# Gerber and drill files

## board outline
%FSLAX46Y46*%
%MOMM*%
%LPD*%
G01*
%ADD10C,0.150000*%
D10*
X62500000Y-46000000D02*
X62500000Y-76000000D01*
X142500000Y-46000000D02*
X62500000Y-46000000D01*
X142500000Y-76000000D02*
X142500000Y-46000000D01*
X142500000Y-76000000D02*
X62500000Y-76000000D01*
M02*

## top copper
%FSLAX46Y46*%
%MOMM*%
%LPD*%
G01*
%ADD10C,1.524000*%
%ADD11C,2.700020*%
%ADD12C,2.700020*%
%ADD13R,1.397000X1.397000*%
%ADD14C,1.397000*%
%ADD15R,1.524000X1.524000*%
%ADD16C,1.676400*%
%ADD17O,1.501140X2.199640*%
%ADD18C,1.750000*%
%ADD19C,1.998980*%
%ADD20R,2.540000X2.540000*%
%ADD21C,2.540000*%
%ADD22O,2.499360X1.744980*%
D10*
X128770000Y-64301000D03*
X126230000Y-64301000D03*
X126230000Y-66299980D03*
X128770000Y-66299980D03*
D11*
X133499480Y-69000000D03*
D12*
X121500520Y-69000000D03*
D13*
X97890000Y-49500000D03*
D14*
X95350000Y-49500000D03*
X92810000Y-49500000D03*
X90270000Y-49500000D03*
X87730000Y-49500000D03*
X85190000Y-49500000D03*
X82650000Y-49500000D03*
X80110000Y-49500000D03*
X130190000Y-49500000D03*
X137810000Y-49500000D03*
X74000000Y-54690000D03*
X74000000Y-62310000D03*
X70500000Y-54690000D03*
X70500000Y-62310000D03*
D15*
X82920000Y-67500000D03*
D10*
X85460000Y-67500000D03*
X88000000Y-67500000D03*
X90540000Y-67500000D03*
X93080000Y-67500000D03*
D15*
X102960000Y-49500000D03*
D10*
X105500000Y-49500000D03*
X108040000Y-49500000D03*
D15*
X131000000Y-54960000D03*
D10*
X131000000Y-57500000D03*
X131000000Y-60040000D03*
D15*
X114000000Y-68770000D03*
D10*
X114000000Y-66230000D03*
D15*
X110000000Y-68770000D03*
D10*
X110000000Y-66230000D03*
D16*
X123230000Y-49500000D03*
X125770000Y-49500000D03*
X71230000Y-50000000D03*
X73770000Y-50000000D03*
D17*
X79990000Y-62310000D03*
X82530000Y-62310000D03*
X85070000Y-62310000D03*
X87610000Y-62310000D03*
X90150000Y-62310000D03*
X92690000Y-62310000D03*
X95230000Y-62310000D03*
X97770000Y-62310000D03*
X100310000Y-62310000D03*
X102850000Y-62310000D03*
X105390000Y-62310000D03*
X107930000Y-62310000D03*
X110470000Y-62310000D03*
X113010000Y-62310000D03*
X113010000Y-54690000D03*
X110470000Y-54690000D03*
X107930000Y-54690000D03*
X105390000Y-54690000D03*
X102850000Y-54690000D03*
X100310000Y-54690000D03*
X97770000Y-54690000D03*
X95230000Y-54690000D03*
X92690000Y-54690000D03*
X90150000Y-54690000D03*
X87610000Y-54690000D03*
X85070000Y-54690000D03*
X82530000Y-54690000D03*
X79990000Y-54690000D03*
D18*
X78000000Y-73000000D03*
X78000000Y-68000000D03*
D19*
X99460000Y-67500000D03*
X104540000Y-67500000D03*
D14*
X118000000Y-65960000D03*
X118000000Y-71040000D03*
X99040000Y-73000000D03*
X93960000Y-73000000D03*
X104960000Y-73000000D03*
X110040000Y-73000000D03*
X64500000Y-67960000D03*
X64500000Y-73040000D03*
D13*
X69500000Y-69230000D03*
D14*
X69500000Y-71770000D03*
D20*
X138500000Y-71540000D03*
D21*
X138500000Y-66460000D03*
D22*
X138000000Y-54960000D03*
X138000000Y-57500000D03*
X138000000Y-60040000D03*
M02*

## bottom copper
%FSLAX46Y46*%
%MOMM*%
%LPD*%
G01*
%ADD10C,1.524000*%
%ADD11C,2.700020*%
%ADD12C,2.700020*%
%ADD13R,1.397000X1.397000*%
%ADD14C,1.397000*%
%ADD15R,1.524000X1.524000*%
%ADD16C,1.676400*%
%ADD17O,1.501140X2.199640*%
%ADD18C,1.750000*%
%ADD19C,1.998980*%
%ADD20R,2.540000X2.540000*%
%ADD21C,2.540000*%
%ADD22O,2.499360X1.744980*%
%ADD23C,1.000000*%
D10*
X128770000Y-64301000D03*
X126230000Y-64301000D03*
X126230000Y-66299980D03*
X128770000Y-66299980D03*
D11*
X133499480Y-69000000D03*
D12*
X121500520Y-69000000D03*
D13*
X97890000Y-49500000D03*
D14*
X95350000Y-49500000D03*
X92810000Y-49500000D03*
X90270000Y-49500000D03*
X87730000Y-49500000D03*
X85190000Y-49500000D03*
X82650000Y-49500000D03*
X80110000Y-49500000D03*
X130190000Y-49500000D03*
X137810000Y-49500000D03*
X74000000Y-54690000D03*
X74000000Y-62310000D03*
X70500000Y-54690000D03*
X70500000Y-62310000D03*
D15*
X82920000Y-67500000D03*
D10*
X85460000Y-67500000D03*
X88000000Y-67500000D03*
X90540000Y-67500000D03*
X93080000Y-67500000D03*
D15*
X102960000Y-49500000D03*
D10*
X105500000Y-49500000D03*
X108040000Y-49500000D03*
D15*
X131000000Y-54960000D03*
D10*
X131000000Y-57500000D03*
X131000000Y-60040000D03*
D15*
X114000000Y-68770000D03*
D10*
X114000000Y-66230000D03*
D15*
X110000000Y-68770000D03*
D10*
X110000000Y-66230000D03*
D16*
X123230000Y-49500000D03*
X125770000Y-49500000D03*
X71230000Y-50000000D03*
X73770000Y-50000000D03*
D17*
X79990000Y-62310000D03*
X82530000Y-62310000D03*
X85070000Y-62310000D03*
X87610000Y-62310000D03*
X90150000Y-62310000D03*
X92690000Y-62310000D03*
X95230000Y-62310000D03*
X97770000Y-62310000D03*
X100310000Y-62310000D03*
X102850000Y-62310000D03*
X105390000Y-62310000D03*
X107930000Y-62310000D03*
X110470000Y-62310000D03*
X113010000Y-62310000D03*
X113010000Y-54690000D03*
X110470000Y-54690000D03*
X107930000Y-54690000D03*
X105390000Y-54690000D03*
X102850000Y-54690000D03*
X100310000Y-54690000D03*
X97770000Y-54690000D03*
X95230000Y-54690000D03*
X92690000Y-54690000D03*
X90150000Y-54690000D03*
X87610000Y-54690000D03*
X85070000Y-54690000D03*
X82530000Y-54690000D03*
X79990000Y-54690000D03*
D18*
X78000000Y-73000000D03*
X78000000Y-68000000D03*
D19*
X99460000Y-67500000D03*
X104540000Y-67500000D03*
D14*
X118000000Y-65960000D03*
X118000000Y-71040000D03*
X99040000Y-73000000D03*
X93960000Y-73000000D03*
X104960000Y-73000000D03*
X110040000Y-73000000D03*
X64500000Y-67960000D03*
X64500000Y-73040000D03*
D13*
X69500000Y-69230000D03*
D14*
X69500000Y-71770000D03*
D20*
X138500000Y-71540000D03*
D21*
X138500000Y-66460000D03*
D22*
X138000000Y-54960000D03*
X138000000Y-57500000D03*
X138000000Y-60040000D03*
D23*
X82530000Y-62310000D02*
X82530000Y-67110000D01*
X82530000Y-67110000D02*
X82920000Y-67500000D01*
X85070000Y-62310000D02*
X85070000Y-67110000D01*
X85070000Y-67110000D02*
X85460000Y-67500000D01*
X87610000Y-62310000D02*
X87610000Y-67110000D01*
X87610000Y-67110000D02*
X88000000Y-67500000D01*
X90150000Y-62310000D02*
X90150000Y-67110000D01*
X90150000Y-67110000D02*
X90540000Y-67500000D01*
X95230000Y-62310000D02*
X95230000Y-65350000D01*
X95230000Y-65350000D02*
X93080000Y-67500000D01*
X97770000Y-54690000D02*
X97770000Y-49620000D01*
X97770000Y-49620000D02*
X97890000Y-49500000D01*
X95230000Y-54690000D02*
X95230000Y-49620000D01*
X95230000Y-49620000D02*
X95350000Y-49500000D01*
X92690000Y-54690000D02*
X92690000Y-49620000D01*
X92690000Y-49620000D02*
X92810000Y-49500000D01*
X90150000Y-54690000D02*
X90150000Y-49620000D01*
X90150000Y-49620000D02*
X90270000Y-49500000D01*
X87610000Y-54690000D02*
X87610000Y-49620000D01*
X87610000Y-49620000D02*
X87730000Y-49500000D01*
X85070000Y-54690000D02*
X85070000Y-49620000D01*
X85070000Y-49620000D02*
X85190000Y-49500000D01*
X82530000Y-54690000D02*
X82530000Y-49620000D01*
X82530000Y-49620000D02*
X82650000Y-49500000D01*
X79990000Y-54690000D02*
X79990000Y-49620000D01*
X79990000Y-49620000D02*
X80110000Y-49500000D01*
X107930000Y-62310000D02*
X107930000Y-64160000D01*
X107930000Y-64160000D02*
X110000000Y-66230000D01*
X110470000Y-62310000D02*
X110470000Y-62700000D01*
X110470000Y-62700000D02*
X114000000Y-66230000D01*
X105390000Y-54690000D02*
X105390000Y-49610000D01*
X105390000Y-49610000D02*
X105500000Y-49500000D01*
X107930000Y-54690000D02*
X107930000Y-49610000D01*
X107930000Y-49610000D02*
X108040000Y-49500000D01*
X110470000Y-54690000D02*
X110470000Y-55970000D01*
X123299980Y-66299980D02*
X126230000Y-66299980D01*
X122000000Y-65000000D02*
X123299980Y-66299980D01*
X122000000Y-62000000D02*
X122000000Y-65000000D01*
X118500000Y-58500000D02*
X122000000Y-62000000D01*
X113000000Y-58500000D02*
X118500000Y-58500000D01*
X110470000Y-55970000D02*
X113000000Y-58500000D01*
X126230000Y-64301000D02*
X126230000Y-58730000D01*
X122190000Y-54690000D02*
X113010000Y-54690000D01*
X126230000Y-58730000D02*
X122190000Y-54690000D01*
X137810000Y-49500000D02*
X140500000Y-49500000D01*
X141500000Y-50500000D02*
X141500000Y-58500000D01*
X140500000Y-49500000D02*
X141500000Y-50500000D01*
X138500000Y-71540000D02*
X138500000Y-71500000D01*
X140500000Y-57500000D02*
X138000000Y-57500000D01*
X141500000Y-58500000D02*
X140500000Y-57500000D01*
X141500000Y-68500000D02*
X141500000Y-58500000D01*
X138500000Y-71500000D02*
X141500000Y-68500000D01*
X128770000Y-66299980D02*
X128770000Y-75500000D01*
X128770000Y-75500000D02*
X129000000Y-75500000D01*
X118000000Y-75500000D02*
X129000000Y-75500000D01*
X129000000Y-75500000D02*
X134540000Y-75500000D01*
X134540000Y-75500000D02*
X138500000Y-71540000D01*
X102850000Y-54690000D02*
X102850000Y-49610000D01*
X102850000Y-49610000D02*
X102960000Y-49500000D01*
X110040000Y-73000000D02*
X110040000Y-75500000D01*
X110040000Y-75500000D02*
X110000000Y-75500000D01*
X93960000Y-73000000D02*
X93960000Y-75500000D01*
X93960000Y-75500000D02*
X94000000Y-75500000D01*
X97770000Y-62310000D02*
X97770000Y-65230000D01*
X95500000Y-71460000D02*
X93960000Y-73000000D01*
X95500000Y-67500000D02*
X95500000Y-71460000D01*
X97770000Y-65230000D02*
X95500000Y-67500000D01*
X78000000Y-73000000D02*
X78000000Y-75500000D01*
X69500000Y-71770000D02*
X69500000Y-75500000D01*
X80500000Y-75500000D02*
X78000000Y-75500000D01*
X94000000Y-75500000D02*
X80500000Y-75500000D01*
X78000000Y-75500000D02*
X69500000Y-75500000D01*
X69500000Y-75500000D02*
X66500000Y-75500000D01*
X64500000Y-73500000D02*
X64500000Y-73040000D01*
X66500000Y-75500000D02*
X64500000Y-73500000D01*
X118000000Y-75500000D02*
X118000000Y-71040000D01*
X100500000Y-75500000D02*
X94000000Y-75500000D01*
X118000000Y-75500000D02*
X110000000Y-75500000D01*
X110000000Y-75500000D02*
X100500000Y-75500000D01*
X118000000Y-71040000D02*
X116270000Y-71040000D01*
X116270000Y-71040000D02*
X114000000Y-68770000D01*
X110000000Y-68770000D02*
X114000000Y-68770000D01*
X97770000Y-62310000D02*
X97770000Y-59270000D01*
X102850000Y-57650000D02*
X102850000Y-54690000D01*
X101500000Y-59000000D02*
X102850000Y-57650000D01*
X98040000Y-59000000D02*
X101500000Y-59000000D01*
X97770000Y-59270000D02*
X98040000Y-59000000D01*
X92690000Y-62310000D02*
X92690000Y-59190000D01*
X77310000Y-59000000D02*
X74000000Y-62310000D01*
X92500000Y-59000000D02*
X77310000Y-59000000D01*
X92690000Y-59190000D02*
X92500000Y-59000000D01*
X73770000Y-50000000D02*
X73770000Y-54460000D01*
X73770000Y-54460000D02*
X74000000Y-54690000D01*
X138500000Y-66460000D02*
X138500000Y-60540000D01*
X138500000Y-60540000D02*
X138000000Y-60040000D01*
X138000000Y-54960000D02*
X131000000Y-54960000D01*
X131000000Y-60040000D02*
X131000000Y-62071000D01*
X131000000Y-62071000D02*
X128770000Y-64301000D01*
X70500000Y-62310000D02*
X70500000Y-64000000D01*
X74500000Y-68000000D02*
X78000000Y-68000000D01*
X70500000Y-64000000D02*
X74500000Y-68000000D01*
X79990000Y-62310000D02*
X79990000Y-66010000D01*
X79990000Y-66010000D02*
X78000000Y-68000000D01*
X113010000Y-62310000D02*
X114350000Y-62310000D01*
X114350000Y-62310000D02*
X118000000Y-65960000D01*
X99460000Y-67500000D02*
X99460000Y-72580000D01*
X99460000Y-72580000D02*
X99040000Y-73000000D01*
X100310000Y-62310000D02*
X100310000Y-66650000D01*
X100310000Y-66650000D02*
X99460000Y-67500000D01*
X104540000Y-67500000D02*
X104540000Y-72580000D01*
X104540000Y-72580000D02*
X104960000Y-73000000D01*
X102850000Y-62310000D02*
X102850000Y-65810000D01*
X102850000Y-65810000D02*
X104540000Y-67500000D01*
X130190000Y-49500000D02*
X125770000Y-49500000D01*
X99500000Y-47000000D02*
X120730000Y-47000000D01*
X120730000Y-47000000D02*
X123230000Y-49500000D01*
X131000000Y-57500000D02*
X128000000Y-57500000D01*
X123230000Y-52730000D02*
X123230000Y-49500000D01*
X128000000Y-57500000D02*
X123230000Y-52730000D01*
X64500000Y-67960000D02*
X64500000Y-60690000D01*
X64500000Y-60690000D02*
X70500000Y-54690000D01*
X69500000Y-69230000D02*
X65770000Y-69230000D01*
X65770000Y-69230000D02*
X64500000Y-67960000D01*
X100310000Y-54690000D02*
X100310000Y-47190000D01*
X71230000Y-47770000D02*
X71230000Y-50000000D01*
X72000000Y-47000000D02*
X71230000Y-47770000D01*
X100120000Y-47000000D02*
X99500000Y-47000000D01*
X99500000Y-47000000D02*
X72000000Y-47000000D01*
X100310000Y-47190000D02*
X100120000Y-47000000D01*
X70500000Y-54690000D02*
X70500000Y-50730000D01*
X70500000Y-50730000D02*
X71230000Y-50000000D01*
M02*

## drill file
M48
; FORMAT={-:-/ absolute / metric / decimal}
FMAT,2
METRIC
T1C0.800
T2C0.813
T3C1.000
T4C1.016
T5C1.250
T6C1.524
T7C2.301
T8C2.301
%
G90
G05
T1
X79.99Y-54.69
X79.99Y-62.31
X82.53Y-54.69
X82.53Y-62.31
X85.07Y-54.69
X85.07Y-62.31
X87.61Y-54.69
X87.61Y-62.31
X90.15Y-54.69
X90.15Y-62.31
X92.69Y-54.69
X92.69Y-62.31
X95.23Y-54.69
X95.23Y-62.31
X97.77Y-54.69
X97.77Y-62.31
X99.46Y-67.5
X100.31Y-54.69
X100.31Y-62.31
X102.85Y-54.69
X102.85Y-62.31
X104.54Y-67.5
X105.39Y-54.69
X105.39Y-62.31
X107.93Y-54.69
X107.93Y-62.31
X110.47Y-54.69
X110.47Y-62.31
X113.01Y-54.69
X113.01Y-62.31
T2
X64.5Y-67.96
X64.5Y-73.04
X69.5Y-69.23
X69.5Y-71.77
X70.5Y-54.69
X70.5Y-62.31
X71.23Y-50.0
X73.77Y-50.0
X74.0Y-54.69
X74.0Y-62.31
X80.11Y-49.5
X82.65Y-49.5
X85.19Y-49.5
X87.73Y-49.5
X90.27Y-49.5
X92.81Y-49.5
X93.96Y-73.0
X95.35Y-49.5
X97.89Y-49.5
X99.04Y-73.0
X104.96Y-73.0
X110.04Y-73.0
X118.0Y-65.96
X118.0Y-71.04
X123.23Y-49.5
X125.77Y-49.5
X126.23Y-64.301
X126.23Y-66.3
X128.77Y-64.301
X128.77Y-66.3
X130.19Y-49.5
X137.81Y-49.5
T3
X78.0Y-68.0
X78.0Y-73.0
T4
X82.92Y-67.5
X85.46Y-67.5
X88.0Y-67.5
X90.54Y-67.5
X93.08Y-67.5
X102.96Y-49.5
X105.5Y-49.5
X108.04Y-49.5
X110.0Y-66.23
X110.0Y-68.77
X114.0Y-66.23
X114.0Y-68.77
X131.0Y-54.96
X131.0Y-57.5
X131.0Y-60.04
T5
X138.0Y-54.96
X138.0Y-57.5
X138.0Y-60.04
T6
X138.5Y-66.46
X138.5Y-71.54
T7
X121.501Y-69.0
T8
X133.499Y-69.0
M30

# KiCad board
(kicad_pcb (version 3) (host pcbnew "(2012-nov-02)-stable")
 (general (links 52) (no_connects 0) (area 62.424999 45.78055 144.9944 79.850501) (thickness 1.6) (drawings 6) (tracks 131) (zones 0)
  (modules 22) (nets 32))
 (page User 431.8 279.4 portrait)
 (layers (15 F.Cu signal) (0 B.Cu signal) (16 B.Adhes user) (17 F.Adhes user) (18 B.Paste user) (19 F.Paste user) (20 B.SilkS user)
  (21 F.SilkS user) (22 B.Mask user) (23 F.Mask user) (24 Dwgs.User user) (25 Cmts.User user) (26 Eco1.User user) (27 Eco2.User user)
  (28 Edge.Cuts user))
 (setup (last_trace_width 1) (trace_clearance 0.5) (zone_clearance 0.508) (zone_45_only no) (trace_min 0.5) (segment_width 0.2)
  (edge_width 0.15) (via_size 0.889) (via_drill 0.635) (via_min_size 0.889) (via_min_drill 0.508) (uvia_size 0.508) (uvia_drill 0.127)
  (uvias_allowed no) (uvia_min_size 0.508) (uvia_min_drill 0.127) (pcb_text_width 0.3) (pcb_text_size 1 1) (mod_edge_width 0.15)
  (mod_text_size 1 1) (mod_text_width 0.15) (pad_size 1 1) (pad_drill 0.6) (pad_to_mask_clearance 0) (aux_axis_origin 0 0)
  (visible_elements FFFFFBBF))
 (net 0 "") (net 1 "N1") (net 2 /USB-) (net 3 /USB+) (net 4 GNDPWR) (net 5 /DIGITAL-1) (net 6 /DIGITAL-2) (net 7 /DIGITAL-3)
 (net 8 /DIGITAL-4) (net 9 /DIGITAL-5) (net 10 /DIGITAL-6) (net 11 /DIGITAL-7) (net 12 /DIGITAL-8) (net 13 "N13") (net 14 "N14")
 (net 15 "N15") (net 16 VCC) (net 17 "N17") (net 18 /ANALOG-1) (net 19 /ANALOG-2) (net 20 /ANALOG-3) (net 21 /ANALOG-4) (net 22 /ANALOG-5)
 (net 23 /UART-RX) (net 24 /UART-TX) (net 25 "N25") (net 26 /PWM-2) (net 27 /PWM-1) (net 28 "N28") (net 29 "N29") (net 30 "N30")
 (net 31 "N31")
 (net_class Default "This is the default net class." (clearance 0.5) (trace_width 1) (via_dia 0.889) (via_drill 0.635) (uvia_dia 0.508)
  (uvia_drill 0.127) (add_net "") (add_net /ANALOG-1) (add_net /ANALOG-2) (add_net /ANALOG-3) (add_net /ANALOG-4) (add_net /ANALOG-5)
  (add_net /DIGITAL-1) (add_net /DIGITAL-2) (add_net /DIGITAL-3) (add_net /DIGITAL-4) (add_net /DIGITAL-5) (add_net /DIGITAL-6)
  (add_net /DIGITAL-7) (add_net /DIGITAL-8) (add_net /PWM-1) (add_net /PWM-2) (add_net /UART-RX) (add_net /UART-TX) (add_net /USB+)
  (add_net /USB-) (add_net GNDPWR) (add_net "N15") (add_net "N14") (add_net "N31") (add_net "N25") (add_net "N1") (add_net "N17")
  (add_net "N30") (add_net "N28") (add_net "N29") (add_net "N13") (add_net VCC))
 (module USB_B (layer F.Cu) (at 127.5 69)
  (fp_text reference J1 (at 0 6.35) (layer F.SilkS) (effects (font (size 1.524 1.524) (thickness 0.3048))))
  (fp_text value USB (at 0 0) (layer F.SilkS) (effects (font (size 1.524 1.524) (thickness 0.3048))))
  (pad 1 thru_hole circle (at 1.27 -4.699) (size 1.524 1.524) (drill 0.8128) (layers *.Cu *.Mask F.SilkS) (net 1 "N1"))
  (pad 2 thru_hole circle (at -1.27 -4.699) (size 1.524 1.524) (drill 0.8128) (layers *.Cu *.Mask F.SilkS) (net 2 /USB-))
  (pad 3 thru_hole circle (at -1.27 -2.70002) (size 1.524 1.524) (drill 0.8128) (layers *.Cu *.Mask F.SilkS) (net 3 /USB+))
  (pad 4 thru_hole circle (at 1.27 -2.70002) (size 1.524 1.524) (drill 0.8128) (layers *.Cu *.Mask F.SilkS) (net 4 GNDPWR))
  (pad 5 np_thru_hole circle (at 5.99948 0) (size 2.70002 2.70002) (drill 2.30124) (layers *.Cu *.SilkS *.Mask))
  (pad 6 thru_hole circle (at -5.99948 0) (size 2.70002 2.70002) (drill 2.30124) (layers *.Cu *.Mask F.SilkS)))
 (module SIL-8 (layer F.Cu) (at 89 49.5 180)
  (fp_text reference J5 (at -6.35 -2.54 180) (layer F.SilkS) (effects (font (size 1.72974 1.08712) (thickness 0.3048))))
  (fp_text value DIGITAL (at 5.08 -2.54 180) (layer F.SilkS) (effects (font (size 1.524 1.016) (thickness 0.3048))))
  (pad 1 thru_hole rect (at -8.89 0 180) (size 1.397 1.397) (drill 0.8128) (layers *.Cu *.Mask F.SilkS) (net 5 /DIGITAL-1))
  (pad 2 thru_hole circle (at -6.35 0 180) (size 1.397 1.397) (drill 0.8128) (layers *.Cu *.Mask F.SilkS) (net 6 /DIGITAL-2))
  (pad 3 thru_hole circle (at -3.81 0 180) (size 1.397 1.397) (drill 0.8128) (layers *.Cu *.Mask F.SilkS) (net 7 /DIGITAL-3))
  (pad 4 thru_hole circle (at -1.27 0 180) (size 1.397 1.397) (drill 0.8128) (layers *.Cu *.Mask F.SilkS) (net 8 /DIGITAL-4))
  (pad 5 thru_hole circle (at 1.27 0 180) (size 1.397 1.397) (drill 0.8128) (layers *.Cu *.Mask F.SilkS) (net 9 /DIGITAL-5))
  (pad 6 thru_hole circle (at 3.81 0 180) (size 1.397 1.397) (drill 0.8128) (layers *.Cu *.Mask F.SilkS) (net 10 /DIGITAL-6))
  (pad 7 thru_hole circle (at 6.35 0 180) (size 1.397 1.397) (drill 0.8128) (layers *.Cu *.Mask F.SilkS) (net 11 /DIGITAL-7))
  (pad 8 thru_hole circle (at 8.89 0 180) (size 1.397 1.397) (drill 0.8128) (layers *.Cu *.Mask F.SilkS) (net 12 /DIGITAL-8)))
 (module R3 (layer F.Cu) (at 134 49.5) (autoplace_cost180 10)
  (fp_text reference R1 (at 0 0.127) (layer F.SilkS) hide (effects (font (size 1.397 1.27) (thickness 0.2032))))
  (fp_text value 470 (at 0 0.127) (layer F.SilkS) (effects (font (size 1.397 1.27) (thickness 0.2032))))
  (pad 1 thru_hole circle (at -3.81 0) (size 1.397 1.397) (drill 0.8128) (layers *.Cu *.Mask F.SilkS) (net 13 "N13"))
  (pad 2 thru_hole circle (at 3.81 0) (size 1.397 1.397) (drill 0.8128) (layers *.Cu *.Mask F.SilkS) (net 4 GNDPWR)))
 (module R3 (layer F.Cu) (at 74 58.5 270) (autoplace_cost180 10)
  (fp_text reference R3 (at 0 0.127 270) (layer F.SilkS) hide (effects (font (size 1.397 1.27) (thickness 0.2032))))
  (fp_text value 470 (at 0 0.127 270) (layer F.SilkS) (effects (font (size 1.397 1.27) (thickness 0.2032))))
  (pad 1 thru_hole circle (at -3.81 0 270) (size 1.397 1.397) (drill 0.8128) (layers *.Cu *.Mask F.SilkS) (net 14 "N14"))
  (pad 2 thru_hole circle (at 3.81 0 270) (size 1.397 1.397) (drill 0.8128) (layers *.Cu *.Mask F.SilkS) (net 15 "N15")))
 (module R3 (layer F.Cu) (at 70.5 58.5 270) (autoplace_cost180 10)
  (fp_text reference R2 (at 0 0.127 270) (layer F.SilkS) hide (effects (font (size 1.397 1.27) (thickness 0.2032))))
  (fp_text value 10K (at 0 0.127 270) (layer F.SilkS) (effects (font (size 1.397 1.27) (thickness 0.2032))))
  (pad 1 thru_hole circle (at -3.81 0 270) (size 1.397 1.397) (drill 0.8128) (layers *.Cu *.Mask F.SilkS) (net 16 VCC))
  (pad 2 thru_hole circle (at 3.81 0 270) (size 1.397 1.397) (drill 0.8128) (layers *.Cu *.Mask F.SilkS) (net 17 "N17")))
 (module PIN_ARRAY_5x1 (layer F.Cu) (at 88 67.5)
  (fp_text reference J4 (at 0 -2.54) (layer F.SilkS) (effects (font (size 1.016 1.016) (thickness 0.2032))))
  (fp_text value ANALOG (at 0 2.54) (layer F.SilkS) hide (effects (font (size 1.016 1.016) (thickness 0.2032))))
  (pad 1 thru_hole rect (at -5.08 0) (size 1.524 1.524) (drill 1.016) (layers *.Cu *.Mask F.SilkS) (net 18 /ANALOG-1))
  (pad 2 thru_hole circle (at -2.54 0) (size 1.524 1.524) (drill 1.016) (layers *.Cu *.Mask F.SilkS) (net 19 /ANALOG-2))
  (pad 3 thru_hole circle (at 0 0) (size 1.524 1.524) (drill 1.016) (layers *.Cu *.Mask F.SilkS) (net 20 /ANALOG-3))
  (pad 4 thru_hole circle (at 2.54 0) (size 1.524 1.524) (drill 1.016) (layers *.Cu *.Mask F.SilkS) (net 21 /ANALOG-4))
  (pad 5 thru_hole circle (at 5.08 0) (size 1.524 1.524) (drill 1.016) (layers *.Cu *.Mask F.SilkS) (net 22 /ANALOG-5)))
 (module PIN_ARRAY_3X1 (layer F.Cu) (at 105.5 49.5)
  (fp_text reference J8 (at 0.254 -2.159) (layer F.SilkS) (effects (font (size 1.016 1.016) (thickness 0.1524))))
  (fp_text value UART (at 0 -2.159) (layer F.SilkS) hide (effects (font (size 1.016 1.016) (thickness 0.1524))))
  (pad 1 thru_hole rect (at -2.54 0) (size 1.524 1.524) (drill 1.016) (layers *.Cu *.Mask F.SilkS) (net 4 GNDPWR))
  (pad 2 thru_hole circle (at 0 0) (size 1.524 1.524) (drill 1.016) (layers *.Cu *.Mask F.SilkS) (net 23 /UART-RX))
  (pad 3 thru_hole circle (at 2.54 0) (size 1.524 1.524) (drill 1.016) (layers *.Cu *.Mask F.SilkS) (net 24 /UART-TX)))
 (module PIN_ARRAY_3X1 (layer F.Cu) (at 131 57.5 270)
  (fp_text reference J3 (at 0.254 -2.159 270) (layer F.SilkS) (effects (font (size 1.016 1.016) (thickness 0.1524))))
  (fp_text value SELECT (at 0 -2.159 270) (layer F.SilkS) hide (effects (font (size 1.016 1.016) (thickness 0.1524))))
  (pad 1 thru_hole rect (at -2.54 0 270) (size 1.524 1.524) (drill 1.016) (layers *.Cu *.Mask F.SilkS) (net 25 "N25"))
  (pad 2 thru_hole circle (at 0 0 270) (size 1.524 1.524) (drill 1.016) (layers *.Cu *.Mask F.SilkS) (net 16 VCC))
  (pad 3 thru_hole circle (at 2.54 0 270) (size 1.524 1.524) (drill 1.016) (layers *.Cu *.Mask F.SilkS) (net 1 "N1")))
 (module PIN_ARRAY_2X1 (layer F.Cu) (at 114 67.5 90)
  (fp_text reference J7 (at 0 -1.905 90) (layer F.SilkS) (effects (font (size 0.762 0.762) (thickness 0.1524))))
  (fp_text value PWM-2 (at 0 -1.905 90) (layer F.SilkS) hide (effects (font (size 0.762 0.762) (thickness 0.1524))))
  (pad 1 thru_hole rect (at -1.27 0 90) (size 1.524 1.524) (drill 1.016) (layers *.Cu *.Mask F.SilkS) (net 4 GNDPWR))
  (pad 2 thru_hole circle (at 1.27 0 90) (size 1.524 1.524) (drill 1.016) (layers *.Cu *.Mask F.SilkS) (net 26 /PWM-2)))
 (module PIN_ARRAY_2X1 (layer F.Cu) (at 110 67.5 90)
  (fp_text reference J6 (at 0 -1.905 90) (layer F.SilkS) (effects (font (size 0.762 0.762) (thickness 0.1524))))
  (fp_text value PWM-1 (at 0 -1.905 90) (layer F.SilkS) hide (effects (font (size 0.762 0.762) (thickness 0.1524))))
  (pad 1 thru_hole rect (at -1.27 0 90) (size 1.524 1.524) (drill 1.016) (layers *.Cu *.Mask F.SilkS) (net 4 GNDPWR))
  (pad 2 thru_hole circle (at 1.27 0 90) (size 1.524 1.524) (drill 1.016) (layers *.Cu *.Mask F.SilkS) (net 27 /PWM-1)))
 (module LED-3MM (layer F.Cu) (at 124.5 49.5)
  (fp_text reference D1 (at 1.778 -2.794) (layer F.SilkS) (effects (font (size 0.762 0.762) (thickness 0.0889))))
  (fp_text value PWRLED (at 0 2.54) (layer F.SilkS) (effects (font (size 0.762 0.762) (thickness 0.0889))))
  (pad 1 thru_hole circle (at -1.27 0) (size 1.6764 1.6764) (drill 0.8128) (layers *.Cu *.Mask F.SilkS) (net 16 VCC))
  (pad 2 thru_hole circle (at 1.27 0) (size 1.6764 1.6764) (drill 0.8128) (layers *.Cu *.Mask F.SilkS) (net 13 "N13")))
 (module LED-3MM (layer F.Cu) (at 72.5 50)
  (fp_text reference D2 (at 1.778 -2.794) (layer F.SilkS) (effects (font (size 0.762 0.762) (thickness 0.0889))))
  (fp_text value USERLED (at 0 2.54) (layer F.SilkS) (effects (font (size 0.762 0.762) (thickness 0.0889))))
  (pad 1 thru_hole circle (at -1.27 0) (size 1.6764 1.6764) (drill 0.8128) (layers *.Cu *.Mask F.SilkS) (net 16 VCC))
  (pad 2 thru_hole circle (at 1.27 0) (size 1.6764 1.6764) (drill 0.8128) (layers *.Cu *.Mask F.SilkS) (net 14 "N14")))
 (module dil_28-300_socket (layer F.Cu) (at 96.5 58.5)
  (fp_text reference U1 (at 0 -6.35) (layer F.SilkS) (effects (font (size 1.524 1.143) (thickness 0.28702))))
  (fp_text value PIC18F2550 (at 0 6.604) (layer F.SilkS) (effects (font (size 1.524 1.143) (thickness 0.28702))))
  (pad 1 thru_hole oval (at -16.51 3.81) (size 1.50114 2.19964) (drill 0.8001) (layers *.Cu *.Mask F.SilkS) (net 17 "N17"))
  (pad 2 thru_hole oval (at -13.97 3.81) (size 1.50114 2.19964) (drill 0.8001) (layers *.Cu *.Mask F.SilkS) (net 18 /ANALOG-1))
  (pad 3 thru_hole oval (at -11.43 3.81) (size 1.50114 2.19964) (drill 0.8001) (layers *.Cu *.Mask F.SilkS) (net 19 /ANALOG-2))
  (pad 4 thru_hole oval (at -8.89 3.81) (size 1.50114 2.19964) (drill 0.8001) (layers *.Cu *.Mask F.SilkS) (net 20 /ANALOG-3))
  (pad 5 thru_hole oval (at -6.35 3.81) (size 1.50114 2.19964) (drill 0.8001) (layers *.Cu *.Mask F.SilkS) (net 21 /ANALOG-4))
  (pad 6 thru_hole oval (at -3.81 3.81) (size 1.50114 2.19964) (drill 0.8001) (layers *.Cu *.Mask F.SilkS) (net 15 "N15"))
  (pad 7 thru_hole oval (at -1.27 3.81) (size 1.50114 2.19964) (drill 0.8001) (layers *.Cu *.Mask F.SilkS) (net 22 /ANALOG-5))
  (pad 8 thru_hole oval (at 1.27 3.81) (size 1.50114 2.19964) (drill 0.8001) (layers *.Cu *.Mask F.SilkS) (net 4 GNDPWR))
  (pad 9 thru_hole oval (at 3.81 3.81) (size 1.50114 2.19964) (drill 0.8001) (layers *.Cu *.Mask F.SilkS) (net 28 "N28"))
  (pad 10 thru_hole oval (at 6.35 3.81) (size 1.50114 2.19964) (drill 0.8001) (layers *.Cu *.Mask F.SilkS) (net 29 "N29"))
  (pad 11 thru_hole oval (at 8.89 3.81) (size 1.50114 2.19964) (drill 0.8001) (layers *.Cu *.Mask F.SilkS))
  (pad 12 thru_hole oval (at 11.43 3.81) (size 1.50114 2.19964) (drill 0.8001) (layers *.Cu *.Mask F.SilkS) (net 27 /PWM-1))
  (pad 13 thru_hole oval (at 13.97 3.81) (size 1.50114 2.19964) (drill 0.8001) (layers *.Cu *.Mask F.SilkS) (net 26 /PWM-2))
  (pad 14 thru_hole oval (at 16.51 3.81) (size 1.50114 2.19964) (drill 0.8001) (layers *.Cu *.Mask F.SilkS) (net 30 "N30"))
  (pad 15 thru_hole oval (at 16.51 -3.81) (size 1.50114 2.19964) (drill 0.8001) (layers *.Cu *.Mask F.SilkS) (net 2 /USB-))
  (pad 16 thru_hole oval (at 13.97 -3.81) (size 1.50114 2.19964) (drill 0.8001) (layers *.Cu *.Mask F.SilkS) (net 3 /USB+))
  (pad 17 thru_hole oval (at 11.43 -3.81) (size 1.50114 2.19964) (drill 0.8001) (layers *.Cu *.Mask F.SilkS) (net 24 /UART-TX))
  (pad 18 thru_hole oval (at 8.89 -3.81) (size 1.50114 2.19964) (drill 0.8001) (layers *.Cu *.Mask F.SilkS) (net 23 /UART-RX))
  (pad 19 thru_hole oval (at 6.35 -3.81) (size 1.50114 2.19964) (drill 0.8001) (layers *.Cu *.Mask F.SilkS) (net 4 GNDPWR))
  (pad 20 thru_hole oval (at 3.81 -3.81) (size 1.50114 2.19964) (drill 0.8001) (layers *.Cu *.Mask F.SilkS) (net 16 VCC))
  (pad 21 thru_hole oval (at 1.27 -3.81) (size 1.50114 2.19964) (drill 0.8001) (layers *.Cu *.Mask F.SilkS) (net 5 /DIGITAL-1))
  (pad 22 thru_hole oval (at -1.27 -3.81) (size 1.50114 2.19964) (drill 0.8001) (layers *.Cu *.Mask F.SilkS) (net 6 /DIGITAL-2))
  (pad 23 thru_hole oval (at -3.81 -3.81) (size 1.50114 2.19964) (drill 0.8001) (layers *.Cu *.Mask F.SilkS) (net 7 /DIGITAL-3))
  (pad 24 thru_hole oval (at -6.35 -3.81) (size 1.50114 2.19964) (drill 0.8001) (layers *.Cu *.Mask F.SilkS) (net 8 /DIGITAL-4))
  (pad 25 thru_hole oval (at -8.89 -3.81) (size 1.50114 2.19964) (drill 0.8001) (layers *.Cu *.Mask F.SilkS) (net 9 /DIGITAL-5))
  (pad 26 thru_hole oval (at -11.43 -3.81) (size 1.50114 2.19964) (drill 0.8001) (layers *.Cu *.Mask F.SilkS) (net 10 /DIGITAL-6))
  (pad 27 thru_hole oval (at -13.97 -3.81) (size 1.50114 2.19964) (drill 0.8001) (layers *.Cu *.Mask F.SilkS) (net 11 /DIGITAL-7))
  (pad 28 thru_hole oval (at -16.51 -3.81) (size 1.50114 2.19964) (drill 0.8001) (layers *.Cu *.Mask F.SilkS) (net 12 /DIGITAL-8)))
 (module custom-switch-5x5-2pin (layer F.Cu) (at 78 70.5 90)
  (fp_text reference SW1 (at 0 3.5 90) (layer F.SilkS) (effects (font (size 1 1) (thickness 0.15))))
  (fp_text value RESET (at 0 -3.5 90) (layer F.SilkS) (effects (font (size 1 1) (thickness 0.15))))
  (pad 1 thru_hole circle (at -2.5 0 90) (size 1.75 1.75) (drill 1) (layers *.Cu *.Mask F.SilkS) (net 4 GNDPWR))
  (pad 2 thru_hole circle (at 2.5 0 90) (size 1.75 1.75) (drill 1) (layers *.Cu *.Mask F.SilkS) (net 17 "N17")))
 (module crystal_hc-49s (layer F.Cu) (at 102 67.5) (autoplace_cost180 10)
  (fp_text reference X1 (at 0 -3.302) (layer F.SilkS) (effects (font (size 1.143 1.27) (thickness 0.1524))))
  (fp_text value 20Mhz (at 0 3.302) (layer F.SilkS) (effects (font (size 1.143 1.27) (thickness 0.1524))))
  (pad 1 thru_hole circle (at -2.54 0) (size 1.99898 1.99898) (drill 0.8001) (layers *.Cu *.Mask F.SilkS) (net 28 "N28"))
  (pad 2 thru_hole circle (at 2.54 0) (size 1.99898 1.99898) (drill 0.8001) (layers *.Cu *.Mask F.SilkS) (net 29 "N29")))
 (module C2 (layer F.Cu) (at 118 68.5 270)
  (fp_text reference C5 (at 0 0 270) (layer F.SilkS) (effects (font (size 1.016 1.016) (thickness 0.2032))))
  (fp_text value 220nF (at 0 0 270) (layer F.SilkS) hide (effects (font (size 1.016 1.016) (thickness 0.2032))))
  (pad 1 thru_hole circle (at -2.54 0 270) (size 1.397 1.397) (drill 0.8128) (layers *.Cu *.Mask F.SilkS) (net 30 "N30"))
  (pad 2 thru_hole circle (at 2.54 0 270) (size 1.397 1.397) (drill 0.8128) (layers *.Cu *.Mask F.SilkS) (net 4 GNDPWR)))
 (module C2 (layer F.Cu) (at 96.5 73 180)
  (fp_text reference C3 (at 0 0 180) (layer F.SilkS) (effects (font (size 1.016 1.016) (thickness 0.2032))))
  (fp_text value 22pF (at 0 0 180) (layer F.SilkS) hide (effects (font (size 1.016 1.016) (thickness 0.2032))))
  (pad 1 thru_hole circle (at -2.54 0 180) (size 1.397 1.397) (drill 0.8128) (layers *.Cu *.Mask F.SilkS) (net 28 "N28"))
  (pad 2 thru_hole circle (at 2.54 0 180) (size 1.397 1.397) (drill 0.8128) (layers *.Cu *.Mask F.SilkS) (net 4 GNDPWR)))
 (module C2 (layer F.Cu) (at 107.5 73)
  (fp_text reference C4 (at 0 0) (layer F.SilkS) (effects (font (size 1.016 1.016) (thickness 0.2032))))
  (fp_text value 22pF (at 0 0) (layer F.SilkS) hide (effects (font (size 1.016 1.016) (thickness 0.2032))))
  (pad 1 thru_hole circle (at -2.54 0) (size 1.397 1.397) (drill 0.8128) (layers *.Cu *.Mask F.SilkS) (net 29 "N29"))
  (pad 2 thru_hole circle (at 2.54 0) (size 1.397 1.397) (drill 0.8128) (layers *.Cu *.Mask F.SilkS) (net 4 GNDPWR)))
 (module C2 (layer F.Cu) (at 64.5 70.5 270)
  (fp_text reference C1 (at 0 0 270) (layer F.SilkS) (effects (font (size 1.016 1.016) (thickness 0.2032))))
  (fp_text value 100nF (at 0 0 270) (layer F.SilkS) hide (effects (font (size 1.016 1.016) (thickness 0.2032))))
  (pad 1 thru_hole circle (at -2.54 0 270) (size 1.397 1.397) (drill 0.8128) (layers *.Cu *.Mask F.SilkS) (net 16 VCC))
  (pad 2 thru_hole circle (at 2.54 0 270) (size 1.397 1.397) (drill 0.8128) (layers *.Cu *.Mask F.SilkS) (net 4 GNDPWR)))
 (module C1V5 (layer F.Cu) (at 69.5 70.5 270)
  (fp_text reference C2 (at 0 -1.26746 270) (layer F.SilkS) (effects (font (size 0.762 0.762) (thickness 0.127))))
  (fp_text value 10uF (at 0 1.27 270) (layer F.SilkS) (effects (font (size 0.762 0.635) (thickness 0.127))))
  (pad 1 thru_hole rect (at -1.27 0 270) (size 1.397 1.397) (drill 0.8128) (layers *.Cu *.Mask F.SilkS) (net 16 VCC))
  (pad 2 thru_hole circle (at 1.27 0 270) (size 1.397 1.397) (drill 0.8128) (layers *.Cu *.Mask F.SilkS) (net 4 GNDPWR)))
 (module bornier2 (layer F.Cu) (at 138.5 69 90)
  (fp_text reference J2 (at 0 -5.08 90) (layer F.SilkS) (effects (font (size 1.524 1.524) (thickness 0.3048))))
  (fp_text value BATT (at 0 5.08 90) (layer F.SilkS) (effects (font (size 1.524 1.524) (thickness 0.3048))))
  (pad 1 thru_hole rect (at -2.54 0 90) (size 2.54 2.54) (drill 1.524) (layers *.Cu *.Mask F.SilkS) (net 4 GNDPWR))
  (pad 2 thru_hole circle (at 2.54 0 90) (size 2.54 2.54) (drill 1.524) (layers *.Cu *.Mask F.SilkS) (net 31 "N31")))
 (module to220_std (layer F.Cu) (at 138 57.5 90)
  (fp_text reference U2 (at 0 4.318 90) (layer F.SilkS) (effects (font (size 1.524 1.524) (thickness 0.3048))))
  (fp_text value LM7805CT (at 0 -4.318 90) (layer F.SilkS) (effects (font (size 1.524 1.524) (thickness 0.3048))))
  (pad 3 thru_hole oval (at 2.54 0 90) (size 1.74498 2.49936) (drill 1.24968) (layers *.Cu *.Mask F.SilkS) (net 25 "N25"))
  (pad 2 thru_hole oval (at 0 0 90) (size 1.74498 2.49936) (drill 1.24968) (layers *.Cu *.Mask F.SilkS) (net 4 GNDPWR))
  (pad 1 thru_hole oval (at -2.54 0 90) (size 1.74498 2.49936) (drill 1.24968) (layers *.Cu *.Mask F.SilkS) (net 31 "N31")))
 (gr_line (start 62.5 46) (end 62.5 76) (angle 90) (layer Edge.Cuts) (width 0.15))
 (gr_line (start 142.5 46) (end 62.5 46) (angle 90) (layer Edge.Cuts) (width 0.15))
 (gr_line (start 142.5 76) (end 142.5 46) (angle 90) (layer Edge.Cuts) (width 0.15))
 (gr_line (start 142.5 76) (end 62.5 76) (angle 90) (layer Edge.Cuts) (width 0.15))
 (segment (start 82.53 62.31) (end 82.53 67.11) (width 1) (layer B.Cu) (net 18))
 (segment (start 82.53 67.11) (end 82.92 67.5) (width 1) (layer B.Cu) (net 18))
 (segment (start 85.07 62.31) (end 85.07 67.11) (width 1) (layer B.Cu) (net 19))
 (segment (start 85.07 67.11) (end 85.46 67.5) (width 1) (layer B.Cu) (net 19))
 (segment (start 87.61 62.31) (end 87.61 67.11) (width 1) (layer B.Cu) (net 20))
 (segment (start 87.61 67.11) (end 88 67.5) (width 1) (layer B.Cu) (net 20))
 (segment (start 90.15 62.31) (end 90.15 67.11) (width 1) (layer B.Cu) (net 21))
 (segment (start 90.15 67.11) (end 90.54 67.5) (width 1) (layer B.Cu) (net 21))
 (segment (start 95.23 62.31) (end 95.23 65.35) (width 1) (layer B.Cu) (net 22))
 (segment (start 95.23 65.35) (end 93.08 67.5) (width 1) (layer B.Cu) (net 22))
 (segment (start 97.77 54.69) (end 97.77 49.62) (width 1) (layer B.Cu) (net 5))
 (segment (start 97.77 49.62) (end 97.89 49.5) (width 1) (layer B.Cu) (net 5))
 (segment (start 95.23 54.69) (end 95.23 49.62) (width 1) (layer B.Cu) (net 6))
 (segment (start 95.23 49.62) (end 95.35 49.5) (width 1) (layer B.Cu) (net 6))
 (segment (start 92.69 54.69) (end 92.69 49.62) (width 1) (layer B.Cu) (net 7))
 (segment (start 92.69 49.62) (end 92.81 49.5) (width 1) (layer B.Cu) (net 7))
 (segment (start 90.15 54.69) (end 90.15 49.62) (width 1) (layer B.Cu) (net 8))
 (segment (start 90.15 49.62) (end 90.27 49.5) (width 1) (layer B.Cu) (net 8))
 (segment (start 87.61 54.69) (end 87.61 49.62) (width 1) (layer B.Cu) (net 9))
 (segment (start 87.61 49.62) (end 87.73 49.5) (width 1) (layer B.Cu) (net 9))
 (segment (start 85.07 54.69) (end 85.07 49.62) (width 1) (layer B.Cu) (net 10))
 (segment (start 85.07 49.62) (end 85.19 49.5) (width 1) (layer B.Cu) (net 10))
 (segment (start 82.53 54.69) (end 82.53 49.62) (width 1) (layer B.Cu) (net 11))
 (segment (start 82.53 49.62) (end 82.65 49.5) (width 1) (layer B.Cu) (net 11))
 (segment (start 79.99 54.69) (end 79.99 49.62) (width 1) (layer B.Cu) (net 12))
 (segment (start 79.99 49.62) (end 80.11 49.5) (width 1) (layer B.Cu) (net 12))
 (segment (start 107.93 62.31) (end 107.93 64.16) (width 1) (layer B.Cu) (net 27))
 (segment (start 107.93 64.16) (end 110 66.23) (width 1) (layer B.Cu) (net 27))
 (segment (start 110.47 62.31) (end 110.47 62.7) (width 1) (layer B.Cu) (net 26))
 (segment (start 110.47 62.7) (end 114 66.23) (width 1) (layer B.Cu) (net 26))
 (segment (start 105.39 54.69) (end 105.39 49.61) (width 1) (layer B.Cu) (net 23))
 (segment (start 105.39 49.61) (end 105.5 49.5) (width 1) (layer B.Cu) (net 23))
 (segment (start 107.93 54.69) (end 107.93 49.61) (width 1) (layer B.Cu) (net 24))
 (segment (start 107.93 49.61) (end 108.04 49.5) (width 1) (layer B.Cu) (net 24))
 (segment (start 110.47 54.69) (end 110.47 55.97) (width 1) (layer B.Cu) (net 3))
 (segment (start 123.29998 66.29998) (end 126.23 66.29998) (width 1) (layer B.Cu) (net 3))
 (segment (start 122 65) (end 123.29998 66.29998) (width 1) (layer B.Cu) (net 3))
 (segment (start 122 62) (end 122 65) (width 1) (layer B.Cu) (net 3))
 (segment (start 118.5 58.5) (end 122 62) (width 1) (layer B.Cu) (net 3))
 (segment (start 113 58.5) (end 118.5 58.5) (width 1) (layer B.Cu) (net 3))
 (segment (start 110.47 55.97) (end 113 58.5) (width 1) (layer B.Cu) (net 3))
 (segment (start 126.23 64.301) (end 126.23 58.73) (width 1) (layer B.Cu) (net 2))
 (segment (start 122.19 54.69) (end 113.01 54.69) (width 1) (layer B.Cu) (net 2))
 (segment (start 126.23 58.73) (end 122.19 54.69) (width 1) (layer B.Cu) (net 2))
 (segment (start 137.81 49.5) (end 140.5 49.5) (width 1) (layer B.Cu) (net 4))
 (segment (start 141.5 50.5) (end 141.5 58.5) (width 1) (layer B.Cu) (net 4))
 (segment (start 140.5 49.5) (end 141.5 50.5) (width 1) (layer B.Cu) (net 4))
 (segment (start 138.5 71.54) (end 138.5 71.5) (width 1) (layer B.Cu) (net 4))
 (segment (start 140.5 57.5) (end 138 57.5) (width 1) (layer B.Cu) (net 4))
 (segment (start 141.5 58.5) (end 140.5 57.5) (width 1) (layer B.Cu) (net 4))
 (segment (start 141.5 68.5) (end 141.5 58.5) (width 1) (layer B.Cu) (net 4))
 (segment (start 138.5 71.5) (end 141.5 68.5) (width 1) (layer B.Cu) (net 4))
 (segment (start 128.77 66.29998) (end 128.77 75.5) (width 1) (layer B.Cu) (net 4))
 (segment (start 128.77 75.5) (end 129 75.5) (width 1) (layer B.Cu) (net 4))
 (segment (start 118 75.5) (end 129 75.5) (width 1) (layer B.Cu) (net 4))
 (segment (start 129 75.5) (end 134.54 75.5) (width 1) (layer B.Cu) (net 4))
 (segment (start 134.54 75.5) (end 138.5 71.54) (width 1) (layer B.Cu) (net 4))
 (segment (start 102.85 54.69) (end 102.85 49.61) (width 1) (layer B.Cu) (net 4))
 (segment (start 102.85 49.61) (end 102.96 49.5) (width 1) (layer B.Cu) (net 4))
 (segment (start 110.04 73) (end 110.04 75.5) (width 1) (layer B.Cu) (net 4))
 (segment (start 110.04 75.5) (end 110 75.5) (width 1) (layer B.Cu) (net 4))
 (segment (start 93.96 73) (end 93.96 75.5) (width 1) (layer B.Cu) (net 4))
 (segment (start 93.96 75.5) (end 94 75.5) (width 1) (layer B.Cu) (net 4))
 (segment (start 97.77 62.31) (end 97.77 65.23) (width 1) (layer B.Cu) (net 4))
 (segment (start 95.5 71.46) (end 93.96 73) (width 1) (layer B.Cu) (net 4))
 (segment (start 95.5 67.5) (end 95.5 71.46) (width 1) (layer B.Cu) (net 4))
 (segment (start 97.77 65.23) (end 95.5 67.5) (width 1) (layer B.Cu) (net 4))
 (segment (start 78 73) (end 78 75.5) (width 1) (layer B.Cu) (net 4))
 (segment (start 69.5 71.77) (end 69.5 75.5) (width 1) (layer B.Cu) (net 4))
 (segment (start 80.5 75.5) (end 78 75.5) (width 1) (layer B.Cu) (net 4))
 (segment (start 94 75.5) (end 80.5 75.5) (width 1) (layer B.Cu) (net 4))
 (segment (start 78 75.5) (end 69.5 75.5) (width 1) (layer B.Cu) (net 4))
 (segment (start 69.5 75.5) (end 66.5 75.5) (width 1) (layer B.Cu) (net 4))
 (segment (start 64.5 73.5) (end 64.5 73.04) (width 1) (layer B.Cu) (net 4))
 (segment (start 66.5 75.5) (end 64.5 73.5) (width 1) (layer B.Cu) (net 4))
 (segment (start 118 75.5) (end 118 71.04) (width 1) (layer B.Cu) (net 4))
 (segment (start 100.5 75.5) (end 94 75.5) (width 1) (layer B.Cu) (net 4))
 (segment (start 118 75.5) (end 110 75.5) (width 1) (layer B.Cu) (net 4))
 (segment (start 110 75.5) (end 100.5 75.5) (width 1) (layer B.Cu) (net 4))
 (segment (start 118 71.04) (end 116.27 71.04) (width 1) (layer B.Cu) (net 4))
 (segment (start 116.27 71.04) (end 114 68.77) (width 1) (layer B.Cu) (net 4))
 (segment (start 110 68.77) (end 114 68.77) (width 1) (layer B.Cu) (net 4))
 (segment (start 97.77 62.31) (end 97.77 59.27) (width 1) (layer B.Cu) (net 4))
 (segment (start 102.85 57.65) (end 102.85 54.69) (width 1) (layer B.Cu) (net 4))
 (segment (start 101.5 59) (end 102.85 57.65) (width 1) (layer B.Cu) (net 4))
 (segment (start 98.04 59) (end 101.5 59) (width 1) (layer B.Cu) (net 4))
 (segment (start 97.77 59.27) (end 98.04 59) (width 1) (layer B.Cu) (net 4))
 (segment (start 92.69 62.31) (end 92.69 59.19) (width 1) (layer B.Cu) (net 15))
 (segment (start 77.31 59) (end 74 62.31) (width 1) (layer B.Cu) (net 15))
 (segment (start 92.5 59) (end 77.31 59) (width 1) (layer B.Cu) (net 15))
 (segment (start 92.69 59.19) (end 92.5 59) (width 1) (layer B.Cu) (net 15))
 (segment (start 73.77 50) (end 73.77 54.46) (width 1) (layer B.Cu) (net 14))
 (segment (start 73.77 54.46) (end 74 54.69) (width 1) (layer B.Cu) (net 14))
 (segment (start 138.5 66.46) (end 138.5 60.54) (width 1) (layer B.Cu) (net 31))
 (segment (start 138.5 60.54) (end 138 60.04) (width 1) (layer B.Cu) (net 31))
 (segment (start 138 54.96) (end 131 54.96) (width 1) (layer B.Cu) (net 25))
 (segment (start 131 60.04) (end 131 62.071) (width 1) (layer B.Cu) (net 1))
 (segment (start 131 62.071) (end 128.77 64.301) (width 1) (layer B.Cu) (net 1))
 (segment (start 70.5 62.31) (end 70.5 64) (width 1) (layer B.Cu) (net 17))
 (segment (start 74.5 68) (end 78 68) (width 1) (layer B.Cu) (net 17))
 (segment (start 70.5 64) (end 74.5 68) (width 1) (layer B.Cu) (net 17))
 (segment (start 79.99 62.31) (end 79.99 66.01) (width 1) (layer B.Cu) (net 17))
 (segment (start 79.99 66.01) (end 78 68) (width 1) (layer B.Cu) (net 17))
 (segment (start 113.01 62.31) (end 114.35 62.31) (width 1) (layer B.Cu) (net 30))
 (segment (start 114.35 62.31) (end 118 65.96) (width 1) (layer B.Cu) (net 30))
 (segment (start 99.46 67.5) (end 99.46 72.58) (width 1) (layer B.Cu) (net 28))
 (segment (start 99.46 72.58) (end 99.04 73) (width 1) (layer B.Cu) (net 28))
 (segment (start 100.31 62.31) (end 100.31 66.65) (width 1) (layer B.Cu) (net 28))
 (segment (start 100.31 66.65) (end 99.46 67.5) (width 1) (layer B.Cu) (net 28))
 (segment (start 104.54 67.5) (end 104.54 72.58) (width 1) (layer B.Cu) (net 29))
 (segment (start 104.54 72.58) (end 104.96 73) (width 1) (layer B.Cu) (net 29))
 (segment (start 102.85 62.31) (end 102.85 65.81) (width 1) (layer B.Cu) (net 29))
 (segment (start 102.85 65.81) (end 104.54 67.5) (width 1) (layer B.Cu) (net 29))
 (segment (start 130.19 49.5) (end 125.77 49.5) (width 1) (layer B.Cu) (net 13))
 (segment (start 99.5 47) (end 120.73 47) (width 1) (layer B.Cu) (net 16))
 (segment (start 120.73 47) (end 123.23 49.5) (width 1) (layer B.Cu) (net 16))
 (segment (start 131 57.5) (end 128 57.5) (width 1) (layer B.Cu) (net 16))
 (segment (start 123.23 52.73) (end 123.23 49.5) (width 1) (layer B.Cu) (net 16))
 (segment (start 128 57.5) (end 123.23 52.73) (width 1) (layer B.Cu) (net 16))
 (segment (start 64.5 67.96) (end 64.5 60.69) (width 1) (layer B.Cu) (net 16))
 (segment (start 64.5 60.69) (end 70.5 54.69) (width 1) (layer B.Cu) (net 16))
 (segment (start 69.5 69.23) (end 65.77 69.23) (width 1) (layer B.Cu) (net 16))
 (segment (start 65.77 69.23) (end 64.5 67.96) (width 1) (layer B.Cu) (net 16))
 (segment (start 100.31 54.69) (end 100.31 47.19) (width 1) (layer B.Cu) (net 16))
 (segment (start 71.23 47.77) (end 71.23 50) (width 1) (layer B.Cu) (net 16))
 (segment (start 72 47) (end 71.23 47.77) (width 1) (layer B.Cu) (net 16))
 (segment (start 100.12 47) (end 99.5 47) (width 1) (layer B.Cu) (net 16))
 (segment (start 99.5 47) (end 72 47) (width 1) (layer B.Cu) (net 16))
 (segment (start 100.31 47.19) (end 100.12 47) (width 1) (layer B.Cu) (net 16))
 (segment (start 70.5 54.69) (end 70.5 50.73) (width 1) (layer B.Cu) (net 16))
 (segment (start 70.5 50.73) (end 71.23 50) (width 1) (layer B.Cu) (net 16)))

